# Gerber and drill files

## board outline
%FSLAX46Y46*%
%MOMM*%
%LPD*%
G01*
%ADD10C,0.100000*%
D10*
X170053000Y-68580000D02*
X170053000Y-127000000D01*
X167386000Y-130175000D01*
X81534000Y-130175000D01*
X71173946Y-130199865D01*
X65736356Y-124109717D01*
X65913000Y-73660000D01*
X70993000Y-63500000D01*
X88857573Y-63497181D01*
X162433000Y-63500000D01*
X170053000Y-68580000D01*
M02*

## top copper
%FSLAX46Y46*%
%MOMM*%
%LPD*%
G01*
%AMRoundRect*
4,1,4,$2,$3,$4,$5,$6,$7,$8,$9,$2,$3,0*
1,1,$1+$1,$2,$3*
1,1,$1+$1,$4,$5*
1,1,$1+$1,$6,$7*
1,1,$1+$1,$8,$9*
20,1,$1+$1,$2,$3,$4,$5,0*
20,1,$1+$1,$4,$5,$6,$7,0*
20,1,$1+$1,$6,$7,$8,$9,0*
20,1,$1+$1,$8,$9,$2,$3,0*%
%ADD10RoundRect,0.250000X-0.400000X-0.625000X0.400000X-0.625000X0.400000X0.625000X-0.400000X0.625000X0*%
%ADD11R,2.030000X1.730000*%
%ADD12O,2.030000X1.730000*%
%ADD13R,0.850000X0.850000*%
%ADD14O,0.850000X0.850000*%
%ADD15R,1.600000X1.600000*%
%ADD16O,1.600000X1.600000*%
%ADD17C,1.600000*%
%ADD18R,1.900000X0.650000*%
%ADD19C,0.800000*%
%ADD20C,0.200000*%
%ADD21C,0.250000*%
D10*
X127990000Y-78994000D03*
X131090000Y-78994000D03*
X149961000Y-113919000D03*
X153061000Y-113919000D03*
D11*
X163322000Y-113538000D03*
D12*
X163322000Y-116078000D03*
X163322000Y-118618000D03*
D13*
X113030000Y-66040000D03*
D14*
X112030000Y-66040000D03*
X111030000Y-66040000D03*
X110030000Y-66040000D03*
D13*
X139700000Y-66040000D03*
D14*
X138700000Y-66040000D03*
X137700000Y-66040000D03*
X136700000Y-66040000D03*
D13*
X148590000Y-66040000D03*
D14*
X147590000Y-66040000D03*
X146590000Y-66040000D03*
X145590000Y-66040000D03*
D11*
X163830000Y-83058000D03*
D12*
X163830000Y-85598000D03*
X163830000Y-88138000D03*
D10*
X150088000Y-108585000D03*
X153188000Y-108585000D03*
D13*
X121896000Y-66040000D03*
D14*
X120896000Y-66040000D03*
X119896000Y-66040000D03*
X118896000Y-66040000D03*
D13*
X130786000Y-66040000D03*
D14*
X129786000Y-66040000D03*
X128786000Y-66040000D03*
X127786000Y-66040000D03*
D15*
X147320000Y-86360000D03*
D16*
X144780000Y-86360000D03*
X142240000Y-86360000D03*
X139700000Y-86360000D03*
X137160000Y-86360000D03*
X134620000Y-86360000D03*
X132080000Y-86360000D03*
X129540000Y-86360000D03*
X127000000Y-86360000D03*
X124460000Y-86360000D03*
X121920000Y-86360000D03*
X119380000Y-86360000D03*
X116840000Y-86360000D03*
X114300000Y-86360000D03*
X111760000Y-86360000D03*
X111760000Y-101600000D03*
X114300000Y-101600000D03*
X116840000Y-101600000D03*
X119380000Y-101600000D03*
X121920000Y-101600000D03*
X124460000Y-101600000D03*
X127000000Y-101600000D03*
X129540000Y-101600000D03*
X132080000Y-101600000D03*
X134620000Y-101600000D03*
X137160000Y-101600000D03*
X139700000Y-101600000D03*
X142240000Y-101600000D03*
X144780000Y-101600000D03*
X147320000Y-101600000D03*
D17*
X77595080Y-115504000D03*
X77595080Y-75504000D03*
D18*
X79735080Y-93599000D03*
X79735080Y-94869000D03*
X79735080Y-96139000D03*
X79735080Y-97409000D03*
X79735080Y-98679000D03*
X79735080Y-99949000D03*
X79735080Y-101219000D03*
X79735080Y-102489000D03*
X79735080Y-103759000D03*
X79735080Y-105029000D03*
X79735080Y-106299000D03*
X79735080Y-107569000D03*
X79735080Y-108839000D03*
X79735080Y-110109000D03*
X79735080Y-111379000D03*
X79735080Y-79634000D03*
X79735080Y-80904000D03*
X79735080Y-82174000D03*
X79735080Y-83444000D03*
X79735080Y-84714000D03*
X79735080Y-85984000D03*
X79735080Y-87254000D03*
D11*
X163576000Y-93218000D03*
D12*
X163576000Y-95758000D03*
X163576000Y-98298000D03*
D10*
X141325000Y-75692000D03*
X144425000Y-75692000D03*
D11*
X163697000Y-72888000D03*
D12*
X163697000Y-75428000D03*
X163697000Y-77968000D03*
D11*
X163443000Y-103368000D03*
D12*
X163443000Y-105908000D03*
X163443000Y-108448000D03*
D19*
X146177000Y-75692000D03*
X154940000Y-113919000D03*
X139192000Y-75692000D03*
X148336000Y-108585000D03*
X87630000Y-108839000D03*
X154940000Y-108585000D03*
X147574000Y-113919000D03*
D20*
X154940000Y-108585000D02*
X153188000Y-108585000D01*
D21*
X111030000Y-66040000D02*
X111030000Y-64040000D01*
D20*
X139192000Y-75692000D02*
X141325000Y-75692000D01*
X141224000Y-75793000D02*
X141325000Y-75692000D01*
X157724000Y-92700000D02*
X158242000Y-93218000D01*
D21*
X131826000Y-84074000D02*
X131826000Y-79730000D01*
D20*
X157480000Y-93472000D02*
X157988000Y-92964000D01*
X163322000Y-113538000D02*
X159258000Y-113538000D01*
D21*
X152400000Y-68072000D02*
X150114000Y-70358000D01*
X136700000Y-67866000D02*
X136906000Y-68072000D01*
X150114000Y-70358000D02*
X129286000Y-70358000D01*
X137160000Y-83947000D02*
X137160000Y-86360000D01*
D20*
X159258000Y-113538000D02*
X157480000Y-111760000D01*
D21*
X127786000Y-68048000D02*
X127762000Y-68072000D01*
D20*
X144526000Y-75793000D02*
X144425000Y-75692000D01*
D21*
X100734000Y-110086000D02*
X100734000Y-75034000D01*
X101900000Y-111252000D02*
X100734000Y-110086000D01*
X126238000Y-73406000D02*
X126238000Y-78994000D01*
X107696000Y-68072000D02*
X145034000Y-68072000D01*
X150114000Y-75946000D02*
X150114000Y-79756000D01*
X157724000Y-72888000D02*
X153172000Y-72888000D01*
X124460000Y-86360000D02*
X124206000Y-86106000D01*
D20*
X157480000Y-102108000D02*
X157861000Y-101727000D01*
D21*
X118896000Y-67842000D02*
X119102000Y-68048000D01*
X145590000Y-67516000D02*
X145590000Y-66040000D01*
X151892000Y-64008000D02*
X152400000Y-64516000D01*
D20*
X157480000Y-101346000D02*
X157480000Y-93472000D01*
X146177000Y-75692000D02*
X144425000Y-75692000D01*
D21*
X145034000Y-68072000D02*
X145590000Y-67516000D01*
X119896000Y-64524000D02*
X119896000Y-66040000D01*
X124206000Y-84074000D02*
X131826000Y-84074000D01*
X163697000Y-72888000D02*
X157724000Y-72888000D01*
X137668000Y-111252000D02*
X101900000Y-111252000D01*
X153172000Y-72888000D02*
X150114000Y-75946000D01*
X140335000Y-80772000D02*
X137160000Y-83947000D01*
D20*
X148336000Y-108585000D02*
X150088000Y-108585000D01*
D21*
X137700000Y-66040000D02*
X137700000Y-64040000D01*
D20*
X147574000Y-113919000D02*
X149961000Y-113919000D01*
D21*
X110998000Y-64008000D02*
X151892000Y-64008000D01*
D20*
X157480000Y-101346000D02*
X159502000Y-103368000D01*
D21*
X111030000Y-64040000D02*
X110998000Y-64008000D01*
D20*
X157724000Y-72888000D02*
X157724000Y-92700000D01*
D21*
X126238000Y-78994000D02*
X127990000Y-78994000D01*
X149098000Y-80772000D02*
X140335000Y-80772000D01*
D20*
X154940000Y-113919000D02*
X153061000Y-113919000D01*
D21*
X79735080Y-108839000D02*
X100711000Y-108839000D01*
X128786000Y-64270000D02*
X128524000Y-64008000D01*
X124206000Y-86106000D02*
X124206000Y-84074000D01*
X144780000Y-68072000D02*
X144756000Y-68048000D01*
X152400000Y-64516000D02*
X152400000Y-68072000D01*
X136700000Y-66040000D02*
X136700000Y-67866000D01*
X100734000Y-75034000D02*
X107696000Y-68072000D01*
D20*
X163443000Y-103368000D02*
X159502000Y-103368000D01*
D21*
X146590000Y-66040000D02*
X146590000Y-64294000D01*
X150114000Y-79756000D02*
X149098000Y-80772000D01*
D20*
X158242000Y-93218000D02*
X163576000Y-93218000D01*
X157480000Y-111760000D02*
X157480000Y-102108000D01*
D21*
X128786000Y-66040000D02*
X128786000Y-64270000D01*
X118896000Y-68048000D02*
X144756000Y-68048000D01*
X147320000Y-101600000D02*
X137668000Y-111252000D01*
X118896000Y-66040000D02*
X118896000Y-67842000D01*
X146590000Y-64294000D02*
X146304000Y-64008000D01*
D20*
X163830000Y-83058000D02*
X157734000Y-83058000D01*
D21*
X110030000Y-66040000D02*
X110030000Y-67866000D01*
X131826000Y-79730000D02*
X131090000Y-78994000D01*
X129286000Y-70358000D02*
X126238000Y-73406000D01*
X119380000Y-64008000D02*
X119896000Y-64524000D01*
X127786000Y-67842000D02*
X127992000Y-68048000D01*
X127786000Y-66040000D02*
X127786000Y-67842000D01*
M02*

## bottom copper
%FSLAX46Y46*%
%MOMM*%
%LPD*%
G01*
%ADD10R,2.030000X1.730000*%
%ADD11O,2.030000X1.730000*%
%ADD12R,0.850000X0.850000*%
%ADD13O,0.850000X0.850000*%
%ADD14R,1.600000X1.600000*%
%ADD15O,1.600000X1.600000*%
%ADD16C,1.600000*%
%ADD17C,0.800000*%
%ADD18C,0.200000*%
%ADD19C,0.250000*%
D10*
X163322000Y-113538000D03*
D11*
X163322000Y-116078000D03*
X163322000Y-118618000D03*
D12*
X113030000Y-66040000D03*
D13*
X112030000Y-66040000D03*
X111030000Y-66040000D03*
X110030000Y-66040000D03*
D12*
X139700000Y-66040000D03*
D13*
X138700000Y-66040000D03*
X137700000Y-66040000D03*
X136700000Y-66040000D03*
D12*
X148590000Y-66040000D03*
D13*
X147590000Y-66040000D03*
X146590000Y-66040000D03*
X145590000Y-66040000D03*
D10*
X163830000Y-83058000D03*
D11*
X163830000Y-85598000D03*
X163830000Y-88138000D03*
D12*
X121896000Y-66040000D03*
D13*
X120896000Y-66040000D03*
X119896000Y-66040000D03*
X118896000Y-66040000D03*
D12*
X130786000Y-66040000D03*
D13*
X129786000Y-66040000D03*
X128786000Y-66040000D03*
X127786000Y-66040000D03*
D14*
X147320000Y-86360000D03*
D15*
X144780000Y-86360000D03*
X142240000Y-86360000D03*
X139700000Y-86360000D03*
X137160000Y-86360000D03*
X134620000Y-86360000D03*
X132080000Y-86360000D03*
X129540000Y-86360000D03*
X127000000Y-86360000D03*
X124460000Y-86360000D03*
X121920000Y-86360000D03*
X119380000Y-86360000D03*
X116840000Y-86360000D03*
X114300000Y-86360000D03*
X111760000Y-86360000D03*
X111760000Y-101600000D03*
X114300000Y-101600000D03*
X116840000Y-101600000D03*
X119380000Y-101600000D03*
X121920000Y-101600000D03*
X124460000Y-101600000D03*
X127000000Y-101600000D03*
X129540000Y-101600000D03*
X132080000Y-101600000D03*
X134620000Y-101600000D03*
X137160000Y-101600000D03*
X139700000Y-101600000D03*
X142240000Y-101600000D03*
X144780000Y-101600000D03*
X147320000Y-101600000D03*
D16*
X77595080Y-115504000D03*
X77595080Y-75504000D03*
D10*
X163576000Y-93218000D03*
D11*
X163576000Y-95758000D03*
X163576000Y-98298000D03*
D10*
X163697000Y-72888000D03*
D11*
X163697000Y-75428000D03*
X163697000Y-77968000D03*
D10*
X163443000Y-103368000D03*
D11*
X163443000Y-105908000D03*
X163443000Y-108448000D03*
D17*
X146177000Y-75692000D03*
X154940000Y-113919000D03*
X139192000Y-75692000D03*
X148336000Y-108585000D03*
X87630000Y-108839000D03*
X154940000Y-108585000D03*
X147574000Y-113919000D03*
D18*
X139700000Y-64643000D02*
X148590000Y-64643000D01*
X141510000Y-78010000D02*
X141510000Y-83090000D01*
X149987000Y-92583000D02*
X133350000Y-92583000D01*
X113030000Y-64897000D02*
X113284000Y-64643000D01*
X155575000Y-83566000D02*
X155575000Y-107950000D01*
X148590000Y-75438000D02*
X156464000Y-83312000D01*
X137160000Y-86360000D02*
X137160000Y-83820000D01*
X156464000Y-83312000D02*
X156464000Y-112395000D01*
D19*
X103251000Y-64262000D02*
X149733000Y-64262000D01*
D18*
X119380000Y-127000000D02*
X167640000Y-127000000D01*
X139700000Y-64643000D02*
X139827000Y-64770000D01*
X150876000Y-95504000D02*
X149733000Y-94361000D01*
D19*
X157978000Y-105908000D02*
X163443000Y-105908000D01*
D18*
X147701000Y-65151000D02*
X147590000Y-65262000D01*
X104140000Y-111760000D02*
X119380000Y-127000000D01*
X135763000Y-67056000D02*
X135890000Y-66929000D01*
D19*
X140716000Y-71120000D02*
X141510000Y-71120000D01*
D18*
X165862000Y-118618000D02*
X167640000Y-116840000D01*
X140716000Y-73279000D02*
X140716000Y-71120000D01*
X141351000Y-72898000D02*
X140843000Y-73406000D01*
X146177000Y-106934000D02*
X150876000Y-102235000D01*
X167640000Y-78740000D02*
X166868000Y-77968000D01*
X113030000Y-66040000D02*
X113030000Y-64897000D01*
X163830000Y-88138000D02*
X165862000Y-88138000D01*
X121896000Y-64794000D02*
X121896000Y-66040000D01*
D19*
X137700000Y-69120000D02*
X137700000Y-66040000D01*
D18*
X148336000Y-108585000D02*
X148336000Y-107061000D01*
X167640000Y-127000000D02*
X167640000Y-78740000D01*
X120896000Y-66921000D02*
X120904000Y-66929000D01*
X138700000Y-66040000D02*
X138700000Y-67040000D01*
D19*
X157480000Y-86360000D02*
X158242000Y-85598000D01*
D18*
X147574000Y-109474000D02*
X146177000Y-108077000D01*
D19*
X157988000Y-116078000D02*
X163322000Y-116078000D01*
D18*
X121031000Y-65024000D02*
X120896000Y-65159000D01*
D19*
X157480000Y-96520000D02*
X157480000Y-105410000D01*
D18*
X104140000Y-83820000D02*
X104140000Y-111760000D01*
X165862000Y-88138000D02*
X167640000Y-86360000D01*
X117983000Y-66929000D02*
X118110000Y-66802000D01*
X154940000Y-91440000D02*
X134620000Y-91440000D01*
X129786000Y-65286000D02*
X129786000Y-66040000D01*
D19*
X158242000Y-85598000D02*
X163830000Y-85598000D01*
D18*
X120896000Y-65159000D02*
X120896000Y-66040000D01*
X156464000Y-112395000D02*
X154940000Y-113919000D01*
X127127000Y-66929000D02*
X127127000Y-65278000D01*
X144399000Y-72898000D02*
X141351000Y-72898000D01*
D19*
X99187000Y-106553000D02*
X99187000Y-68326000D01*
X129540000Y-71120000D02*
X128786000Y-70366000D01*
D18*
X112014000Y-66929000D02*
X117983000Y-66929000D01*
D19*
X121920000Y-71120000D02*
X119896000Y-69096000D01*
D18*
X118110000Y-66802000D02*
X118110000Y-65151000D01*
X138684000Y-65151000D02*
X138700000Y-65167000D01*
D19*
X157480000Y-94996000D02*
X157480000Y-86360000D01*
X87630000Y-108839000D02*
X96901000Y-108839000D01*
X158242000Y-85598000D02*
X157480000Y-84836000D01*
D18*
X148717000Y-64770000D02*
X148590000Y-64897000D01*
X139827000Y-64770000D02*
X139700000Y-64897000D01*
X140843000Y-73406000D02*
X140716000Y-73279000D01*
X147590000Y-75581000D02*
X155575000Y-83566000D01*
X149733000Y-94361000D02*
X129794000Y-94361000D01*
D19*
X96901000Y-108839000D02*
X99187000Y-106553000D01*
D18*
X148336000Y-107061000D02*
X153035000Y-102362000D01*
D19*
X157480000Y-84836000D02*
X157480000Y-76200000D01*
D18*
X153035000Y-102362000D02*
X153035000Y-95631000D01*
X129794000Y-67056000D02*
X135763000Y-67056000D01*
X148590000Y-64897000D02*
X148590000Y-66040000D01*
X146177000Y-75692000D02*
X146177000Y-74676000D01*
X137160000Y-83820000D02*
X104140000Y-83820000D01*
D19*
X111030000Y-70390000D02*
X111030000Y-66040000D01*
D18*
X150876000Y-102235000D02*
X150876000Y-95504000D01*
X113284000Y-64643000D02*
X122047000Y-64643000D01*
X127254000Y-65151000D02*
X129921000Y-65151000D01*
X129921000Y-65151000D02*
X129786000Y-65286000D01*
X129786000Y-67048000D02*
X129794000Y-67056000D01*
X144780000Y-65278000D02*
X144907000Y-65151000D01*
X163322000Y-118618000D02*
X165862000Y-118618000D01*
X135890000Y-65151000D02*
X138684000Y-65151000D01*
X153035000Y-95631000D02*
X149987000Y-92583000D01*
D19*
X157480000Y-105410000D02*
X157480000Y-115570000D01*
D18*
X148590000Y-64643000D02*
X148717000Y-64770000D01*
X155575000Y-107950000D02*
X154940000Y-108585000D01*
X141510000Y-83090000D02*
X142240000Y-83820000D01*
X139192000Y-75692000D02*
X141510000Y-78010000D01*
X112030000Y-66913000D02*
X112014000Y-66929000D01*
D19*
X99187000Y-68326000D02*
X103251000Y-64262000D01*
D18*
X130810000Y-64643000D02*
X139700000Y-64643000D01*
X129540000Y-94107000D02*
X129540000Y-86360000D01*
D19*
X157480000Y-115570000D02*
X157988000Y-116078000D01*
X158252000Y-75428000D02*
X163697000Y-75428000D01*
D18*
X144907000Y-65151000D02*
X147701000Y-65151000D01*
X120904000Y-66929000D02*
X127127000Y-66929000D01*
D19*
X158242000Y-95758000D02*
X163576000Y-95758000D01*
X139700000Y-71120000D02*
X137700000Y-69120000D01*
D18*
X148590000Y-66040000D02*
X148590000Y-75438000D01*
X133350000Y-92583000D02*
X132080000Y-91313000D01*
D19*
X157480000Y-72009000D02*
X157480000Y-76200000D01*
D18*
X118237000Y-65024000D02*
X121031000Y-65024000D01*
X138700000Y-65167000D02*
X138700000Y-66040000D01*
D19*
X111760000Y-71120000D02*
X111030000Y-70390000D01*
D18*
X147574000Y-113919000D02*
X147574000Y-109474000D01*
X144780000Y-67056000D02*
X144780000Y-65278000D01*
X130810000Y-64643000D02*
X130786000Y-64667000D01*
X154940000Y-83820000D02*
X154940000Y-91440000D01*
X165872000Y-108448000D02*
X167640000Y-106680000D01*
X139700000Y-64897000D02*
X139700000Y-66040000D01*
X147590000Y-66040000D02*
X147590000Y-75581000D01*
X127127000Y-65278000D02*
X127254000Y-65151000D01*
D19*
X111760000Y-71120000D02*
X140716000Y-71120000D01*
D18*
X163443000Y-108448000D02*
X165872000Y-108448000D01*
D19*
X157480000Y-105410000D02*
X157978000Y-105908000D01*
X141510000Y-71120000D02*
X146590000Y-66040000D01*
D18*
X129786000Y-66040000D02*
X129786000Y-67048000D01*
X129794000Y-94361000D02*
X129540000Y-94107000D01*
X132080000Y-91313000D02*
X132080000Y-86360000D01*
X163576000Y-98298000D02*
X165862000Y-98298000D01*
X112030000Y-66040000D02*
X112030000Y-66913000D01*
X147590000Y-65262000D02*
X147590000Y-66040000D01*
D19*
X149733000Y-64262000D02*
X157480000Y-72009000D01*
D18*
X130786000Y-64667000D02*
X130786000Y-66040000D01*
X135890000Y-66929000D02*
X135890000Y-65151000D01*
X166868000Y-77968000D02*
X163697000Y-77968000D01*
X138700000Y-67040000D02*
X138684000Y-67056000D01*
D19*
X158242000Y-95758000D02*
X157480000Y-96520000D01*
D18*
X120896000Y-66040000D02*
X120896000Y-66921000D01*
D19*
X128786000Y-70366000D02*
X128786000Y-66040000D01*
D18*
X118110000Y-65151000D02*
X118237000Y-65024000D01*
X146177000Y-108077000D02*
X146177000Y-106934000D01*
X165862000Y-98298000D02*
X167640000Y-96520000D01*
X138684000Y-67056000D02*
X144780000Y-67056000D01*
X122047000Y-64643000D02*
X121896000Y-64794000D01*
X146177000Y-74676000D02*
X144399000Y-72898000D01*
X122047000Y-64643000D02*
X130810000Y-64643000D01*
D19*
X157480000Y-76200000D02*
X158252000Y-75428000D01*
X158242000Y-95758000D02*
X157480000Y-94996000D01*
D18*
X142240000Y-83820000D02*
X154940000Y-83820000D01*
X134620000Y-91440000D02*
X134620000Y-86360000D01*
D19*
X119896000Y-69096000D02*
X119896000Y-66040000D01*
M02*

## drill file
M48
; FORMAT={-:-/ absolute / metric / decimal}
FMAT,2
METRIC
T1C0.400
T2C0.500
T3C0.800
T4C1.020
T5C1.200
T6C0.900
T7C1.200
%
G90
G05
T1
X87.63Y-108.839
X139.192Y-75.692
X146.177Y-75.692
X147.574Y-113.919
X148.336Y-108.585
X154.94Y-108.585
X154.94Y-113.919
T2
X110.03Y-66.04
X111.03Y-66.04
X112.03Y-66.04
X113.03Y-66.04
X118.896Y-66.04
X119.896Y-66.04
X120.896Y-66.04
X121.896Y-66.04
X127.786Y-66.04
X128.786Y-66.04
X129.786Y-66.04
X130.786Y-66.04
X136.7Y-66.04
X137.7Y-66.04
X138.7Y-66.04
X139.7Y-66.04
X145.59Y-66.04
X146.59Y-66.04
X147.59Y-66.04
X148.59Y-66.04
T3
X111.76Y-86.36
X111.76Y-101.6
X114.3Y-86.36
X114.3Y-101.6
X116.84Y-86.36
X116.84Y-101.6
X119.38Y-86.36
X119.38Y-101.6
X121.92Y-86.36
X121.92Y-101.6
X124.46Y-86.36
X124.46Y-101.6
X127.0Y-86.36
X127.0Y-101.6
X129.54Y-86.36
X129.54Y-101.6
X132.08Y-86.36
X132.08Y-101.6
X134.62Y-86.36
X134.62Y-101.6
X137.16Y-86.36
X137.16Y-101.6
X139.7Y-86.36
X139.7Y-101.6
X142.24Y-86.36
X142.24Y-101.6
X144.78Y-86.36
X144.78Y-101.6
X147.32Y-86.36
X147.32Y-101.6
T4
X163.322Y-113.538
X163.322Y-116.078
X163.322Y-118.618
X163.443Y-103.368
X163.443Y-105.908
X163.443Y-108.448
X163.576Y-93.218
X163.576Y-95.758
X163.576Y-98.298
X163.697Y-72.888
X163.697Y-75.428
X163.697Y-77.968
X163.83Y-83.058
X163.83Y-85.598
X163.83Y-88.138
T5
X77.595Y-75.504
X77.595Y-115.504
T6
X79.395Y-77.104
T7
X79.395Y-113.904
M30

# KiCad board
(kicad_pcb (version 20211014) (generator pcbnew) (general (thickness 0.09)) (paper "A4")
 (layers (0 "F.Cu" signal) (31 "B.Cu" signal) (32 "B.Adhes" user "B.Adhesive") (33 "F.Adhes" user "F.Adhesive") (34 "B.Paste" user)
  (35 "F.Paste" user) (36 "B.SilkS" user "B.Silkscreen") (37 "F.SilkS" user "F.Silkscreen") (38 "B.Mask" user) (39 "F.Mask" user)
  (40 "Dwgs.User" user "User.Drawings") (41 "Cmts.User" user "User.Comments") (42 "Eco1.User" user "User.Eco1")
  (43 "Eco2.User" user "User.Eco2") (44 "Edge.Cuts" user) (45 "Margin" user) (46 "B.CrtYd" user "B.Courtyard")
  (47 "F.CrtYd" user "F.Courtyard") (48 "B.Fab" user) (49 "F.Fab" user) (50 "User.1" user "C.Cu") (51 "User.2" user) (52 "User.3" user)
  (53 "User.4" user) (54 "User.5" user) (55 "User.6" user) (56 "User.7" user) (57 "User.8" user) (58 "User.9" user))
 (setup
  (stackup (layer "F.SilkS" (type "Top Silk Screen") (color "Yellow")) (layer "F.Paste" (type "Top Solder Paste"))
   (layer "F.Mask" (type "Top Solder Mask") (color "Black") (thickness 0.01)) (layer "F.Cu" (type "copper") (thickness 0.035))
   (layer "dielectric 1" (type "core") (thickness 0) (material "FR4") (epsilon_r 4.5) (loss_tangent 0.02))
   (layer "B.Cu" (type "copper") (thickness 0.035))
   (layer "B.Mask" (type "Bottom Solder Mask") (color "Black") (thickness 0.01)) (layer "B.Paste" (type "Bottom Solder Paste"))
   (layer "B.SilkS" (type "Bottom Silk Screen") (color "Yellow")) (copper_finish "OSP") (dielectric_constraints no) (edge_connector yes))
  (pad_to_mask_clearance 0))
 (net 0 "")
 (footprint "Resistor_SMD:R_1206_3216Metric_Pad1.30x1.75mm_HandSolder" (layer "F.Cu") (at 129.54 78.994)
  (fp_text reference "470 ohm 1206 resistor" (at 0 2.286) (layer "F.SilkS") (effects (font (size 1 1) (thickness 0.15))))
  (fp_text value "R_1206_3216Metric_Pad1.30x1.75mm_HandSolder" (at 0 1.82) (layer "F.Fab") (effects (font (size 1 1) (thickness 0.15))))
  (pad "1" smd roundrect (at -1.55 0) (size 1.3 1.75) (layers "F.Cu" "F.Paste" "F.Mask") (roundrect_rratio 0.1923076923))
  (pad "2" smd roundrect (at 1.55 0) (size 1.3 1.75) (layers "F.Cu" "F.Paste" "F.Mask") (roundrect_rratio 0.1923076923)))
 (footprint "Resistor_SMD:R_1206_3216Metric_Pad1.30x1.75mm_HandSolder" (layer "F.Cu") (at 151.511 113.919)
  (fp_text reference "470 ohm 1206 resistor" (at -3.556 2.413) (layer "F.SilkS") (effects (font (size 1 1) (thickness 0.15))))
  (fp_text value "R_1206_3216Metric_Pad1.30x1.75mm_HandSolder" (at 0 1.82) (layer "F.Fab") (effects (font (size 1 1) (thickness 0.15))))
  (pad "1" smd roundrect (at -1.55 0) (size 1.3 1.75) (layers "F.Cu" "F.Paste" "F.Mask") (roundrect_rratio 0.1923076923))
  (pad "2" smd roundrect (at 1.55 0) (size 1.3 1.75) (layers "F.Cu" "F.Paste" "F.Mask") (roundrect_rratio 0.1923076923)))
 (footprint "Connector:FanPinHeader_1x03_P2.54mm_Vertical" (layer "F.Cu") (at 163.322 113.538 -90)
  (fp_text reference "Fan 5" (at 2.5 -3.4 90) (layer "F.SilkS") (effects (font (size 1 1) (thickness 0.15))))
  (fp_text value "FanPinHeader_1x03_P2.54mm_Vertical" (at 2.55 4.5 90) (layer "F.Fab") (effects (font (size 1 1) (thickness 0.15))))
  (pad "1" thru_hole rect (at 0 0) (size 2.03 1.73) (drill 1.02) (layers *.Cu *.Mask))
  (pad "2" thru_hole oval (at 2.54 0) (size 2.03 1.73) (drill 1.02) (layers *.Cu *.Mask))
  (pad "3" thru_hole oval (at 5.08 0) (size 2.03 1.73) (drill 1.02) (layers *.Cu *.Mask)))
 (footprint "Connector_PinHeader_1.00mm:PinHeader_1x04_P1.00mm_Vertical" (layer "F.Cu") (at 113.03 66.04 -90)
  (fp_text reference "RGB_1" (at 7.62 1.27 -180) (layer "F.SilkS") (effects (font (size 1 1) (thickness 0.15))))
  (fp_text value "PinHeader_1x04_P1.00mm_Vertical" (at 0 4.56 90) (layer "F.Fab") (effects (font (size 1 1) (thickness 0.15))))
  (pad "1" thru_hole rect (at 0 0 270) (size 0.85 0.85) (drill 0.5) (layers *.Cu *.Mask))
  (pad "2" thru_hole oval (at 0 1 270) (size 0.85 0.85) (drill 0.5) (layers *.Cu *.Mask))
  (pad "3" thru_hole oval (at 0 2 270) (size 0.85 0.85) (drill 0.5) (layers *.Cu *.Mask))
  (pad "4" thru_hole oval (at 0 3 270) (size 0.85 0.85) (drill 0.5) (layers *.Cu *.Mask)))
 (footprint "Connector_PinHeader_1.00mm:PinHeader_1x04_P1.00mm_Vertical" (layer "F.Cu") (at 139.7 66.04 -90)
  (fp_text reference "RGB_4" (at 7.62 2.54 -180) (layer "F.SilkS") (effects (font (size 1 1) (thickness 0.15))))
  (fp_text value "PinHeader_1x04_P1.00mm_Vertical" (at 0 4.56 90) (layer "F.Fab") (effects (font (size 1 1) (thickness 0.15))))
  (pad "1" thru_hole rect (at 0 0 270) (size 0.85 0.85) (drill 0.5) (layers *.Cu *.Mask))
  (pad "2" thru_hole oval (at 0 1 270) (size 0.85 0.85) (drill 0.5) (layers *.Cu *.Mask))
  (pad "3" thru_hole oval (at 0 2 270) (size 0.85 0.85) (drill 0.5) (layers *.Cu *.Mask))
  (pad "4" thru_hole oval (at 0 3 270) (size 0.85 0.85) (drill 0.5) (layers *.Cu *.Mask)))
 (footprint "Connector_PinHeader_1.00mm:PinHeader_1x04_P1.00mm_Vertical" (layer "F.Cu") (at 148.59 66.04 -90)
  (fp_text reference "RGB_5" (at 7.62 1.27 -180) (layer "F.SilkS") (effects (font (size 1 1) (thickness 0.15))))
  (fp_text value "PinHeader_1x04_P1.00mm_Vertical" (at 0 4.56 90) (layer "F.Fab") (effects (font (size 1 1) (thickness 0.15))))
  (pad "1" thru_hole rect (at 0 0 270) (size 0.85 0.85) (drill 0.5) (layers *.Cu *.Mask))
  (pad "2" thru_hole oval (at 0 1 270) (size 0.85 0.85) (drill 0.5) (layers *.Cu *.Mask))
  (pad "3" thru_hole oval (at 0 2 270) (size 0.85 0.85) (drill 0.5) (layers *.Cu *.Mask))
  (pad "4" thru_hole oval (at 0 3 270) (size 0.85 0.85) (drill 0.5) (layers *.Cu *.Mask)))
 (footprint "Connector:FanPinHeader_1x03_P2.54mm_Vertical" (layer "F.Cu") (at 163.83 83.058 -90)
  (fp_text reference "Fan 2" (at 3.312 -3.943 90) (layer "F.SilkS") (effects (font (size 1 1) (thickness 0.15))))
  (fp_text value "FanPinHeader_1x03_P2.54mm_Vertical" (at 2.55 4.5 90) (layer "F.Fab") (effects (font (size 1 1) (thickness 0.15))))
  (pad "1" thru_hole rect (at 0 0) (size 2.03 1.73) (drill 1.02) (layers *.Cu *.Mask))
  (pad "2" thru_hole oval (at 2.54 0) (size 2.03 1.73) (drill 1.02) (layers *.Cu *.Mask))
  (pad "3" thru_hole oval (at 5.08 0) (size 2.03 1.73) (drill 1.02) (layers *.Cu *.Mask)))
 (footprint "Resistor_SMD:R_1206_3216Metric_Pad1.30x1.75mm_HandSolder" (layer "F.Cu") (at 151.638 108.585)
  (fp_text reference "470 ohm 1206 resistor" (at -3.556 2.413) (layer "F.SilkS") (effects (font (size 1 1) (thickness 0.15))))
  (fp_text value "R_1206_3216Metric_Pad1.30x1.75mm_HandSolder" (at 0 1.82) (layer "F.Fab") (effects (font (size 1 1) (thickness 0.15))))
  (pad "1" smd roundrect (at -1.55 0) (size 1.3 1.75) (layers "F.Cu" "F.Paste" "F.Mask") (roundrect_rratio 0.1923076923))
  (pad "2" smd roundrect (at 1.55 0) (size 1.3 1.75) (layers "F.Cu" "F.Paste" "F.Mask") (roundrect_rratio 0.1923076923)))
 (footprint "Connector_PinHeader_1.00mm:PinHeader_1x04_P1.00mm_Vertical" (layer "F.Cu") (at 121.896 66.04 -90)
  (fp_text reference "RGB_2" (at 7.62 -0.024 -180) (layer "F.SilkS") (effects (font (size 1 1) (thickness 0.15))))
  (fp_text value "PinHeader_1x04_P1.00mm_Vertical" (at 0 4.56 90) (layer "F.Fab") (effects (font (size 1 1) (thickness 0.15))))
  (pad "1" thru_hole rect (at 0 0 270) (size 0.85 0.85) (drill 0.5) (layers *.Cu *.Mask))
  (pad "2" thru_hole oval (at 0 1 270) (size 0.85 0.85) (drill 0.5) (layers *.Cu *.Mask))
  (pad "3" thru_hole oval (at 0 2 270) (size 0.85 0.85) (drill 0.5) (layers *.Cu *.Mask))
  (pad "4" thru_hole oval (at 0 3 270) (size 0.85 0.85) (drill 0.5) (layers *.Cu *.Mask)))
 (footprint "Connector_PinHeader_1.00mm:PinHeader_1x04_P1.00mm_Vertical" (layer "F.Cu") (at 130.786 66.04 -90)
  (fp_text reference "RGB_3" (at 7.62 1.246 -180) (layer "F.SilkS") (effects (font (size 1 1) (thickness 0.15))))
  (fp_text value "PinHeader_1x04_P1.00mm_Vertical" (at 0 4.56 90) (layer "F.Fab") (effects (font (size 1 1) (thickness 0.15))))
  (pad "1" thru_hole rect (at 0 0 270) (size 0.85 0.85) (drill 0.5) (layers *.Cu *.Mask))
  (pad "2" thru_hole oval (at 0 1 270) (size 0.85 0.85) (drill 0.5) (layers *.Cu *.Mask))
  (pad "3" thru_hole oval (at 0 2 270) (size 0.85 0.85) (drill 0.5) (layers *.Cu *.Mask))
  (pad "4" thru_hole oval (at 0 3 270) (size 0.85 0.85) (drill 0.5) (layers *.Cu *.Mask)))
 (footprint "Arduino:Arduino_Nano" (layer "F.Cu") (at 147.32 86.36 -90)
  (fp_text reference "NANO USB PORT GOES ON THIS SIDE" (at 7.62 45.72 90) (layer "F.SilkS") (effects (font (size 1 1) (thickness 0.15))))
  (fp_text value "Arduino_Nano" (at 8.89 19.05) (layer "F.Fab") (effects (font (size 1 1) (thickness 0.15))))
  (pad "1" thru_hole rect locked (at 0 0 270) (size 1.6 1.6) (drill 0.8) (layers *.Cu *.Mask))
  (pad "2" thru_hole oval locked (at 0 2.54 270) (size 1.6 1.6) (drill 0.8) (layers *.Cu *.Mask))
  (pad "3" thru_hole oval locked (at 0 5.08 270) (size 1.6 1.6) (drill 0.8) (layers *.Cu *.Mask))
  (pad "4" thru_hole oval locked (at 0 7.62 270) (size 1.6 1.6) (drill 0.8) (layers *.Cu *.Mask))
  (pad "5" thru_hole oval locked (at 0 10.16 270) (size 1.6 1.6) (drill 0.8) (layers *.Cu *.Mask))
  (pad "6" thru_hole oval locked (at 0 12.7 270) (size 1.6 1.6) (drill 0.8) (layers *.Cu *.Mask))
  (pad "7" thru_hole oval locked (at 0 15.24 270) (size 1.6 1.6) (drill 0.8) (layers *.Cu *.Mask))
  (pad "8" thru_hole oval locked (at 0 17.78 270) (size 1.6 1.6) (drill 0.8) (layers *.Cu *.Mask))
  (pad "9" thru_hole oval locked (at 0 20.32 270) (size 1.6 1.6) (drill 0.8) (layers *.Cu *.Mask))
  (pad "10" thru_hole oval locked (at 0 22.86 270) (size 1.6 1.6) (drill 0.8) (layers *.Cu *.Mask))
  (pad "11" thru_hole oval locked (at 0 25.4 270) (size 1.6 1.6) (drill 0.8) (layers *.Cu *.Mask))
  (pad "12" thru_hole oval locked (at 0 27.94 270) (size 1.6 1.6) (drill 0.8) (layers *.Cu *.Mask))
  (pad "13" thru_hole oval locked (at 0 30.48 270) (size 1.6 1.6) (drill 0.8) (layers *.Cu *.Mask))
  (pad "14" thru_hole oval locked (at 0 33.02 270) (size 1.6 1.6) (drill 0.8) (layers *.Cu *.Mask))
  (pad "15" thru_hole oval locked (at 0 35.56 270) (size 1.6 1.6) (drill 0.8) (layers *.Cu *.Mask))
  (pad "16" thru_hole oval locked (at 15.24 35.56 270) (size 1.6 1.6) (drill 0.8) (layers *.Cu *.Mask))
  (pad "17" thru_hole oval locked (at 15.24 33.02 270) (size 1.6 1.6) (drill 0.8) (layers *.Cu *.Mask))
  (pad "18" thru_hole oval locked (at 15.24 30.48 270) (size 1.6 1.6) (drill 0.8) (layers *.Cu *.Mask))
  (pad "19" thru_hole oval locked (at 15.24 27.94 270) (size 1.6 1.6) (drill 0.8) (layers *.Cu *.Mask))
  (pad "20" thru_hole oval locked (at 15.24 25.4 270) (size 1.6 1.6) (drill 0.8) (layers *.Cu *.Mask))
  (pad "21" thru_hole oval locked (at 15.24 22.86 270) (size 1.6 1.6) (drill 0.8) (layers *.Cu *.Mask))
  (pad "22" thru_hole oval locked (at 15.24 20.32 270) (size 1.6 1.6) (drill 0.8) (layers *.Cu *.Mask))
  (pad "23" thru_hole oval locked (at 15.24 17.78 270) (size 1.6 1.6) (drill 0.8) (layers *.Cu *.Mask))
  (pad "24" thru_hole oval locked (at 15.24 15.24 270) (size 1.6 1.6) (drill 0.8) (layers *.Cu *.Mask))
  (pad "25" thru_hole oval locked (at 15.24 12.7 270) (size 1.6 1.6) (drill 0.8) (layers *.Cu *.Mask))
  (pad "26" thru_hole oval locked (at 15.24 10.16 270) (size 1.6 1.6) (drill 0.8) (layers *.Cu *.Mask))
  (pad "27" thru_hole oval locked (at 15.24 7.62 270) (size 1.6 1.6) (drill 0.8) (layers *.Cu *.Mask))
  (pad "28" thru_hole oval locked (at 15.24 5.08 270) (size 1.6 1.6) (drill 0.8) (layers *.Cu *.Mask))
  (pad "29" thru_hole oval locked (at 15.24 2.54 270) (size 1.6 1.6) (drill 0.8) (layers *.Cu *.Mask))
  (pad "30" thru_hole oval locked (at 15.24 0 270) (size 1.6 1.6) (drill 0.8) (layers *.Cu *.Mask)))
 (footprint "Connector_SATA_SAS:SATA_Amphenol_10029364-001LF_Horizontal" (layer "F.Cu") (at 78.74 95.504 90)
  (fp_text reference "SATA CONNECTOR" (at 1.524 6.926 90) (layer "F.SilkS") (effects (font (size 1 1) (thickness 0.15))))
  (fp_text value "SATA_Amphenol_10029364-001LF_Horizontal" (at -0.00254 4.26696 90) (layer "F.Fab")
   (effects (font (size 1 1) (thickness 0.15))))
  (pad "" np_thru_hole circle (at -18.4 0.65508 90) (size 1.2 1.2) (drill 1.2) (layers *.Mask "B.Cu"))
  (pad "" np_thru_hole circle (at 18.4 0.65508 90) (size 0.9 0.9) (drill 0.9) (layers *.Mask "B.Cu"))
  (pad "MP" thru_hole circle (at -20 -1.14492 90) (size 1.6 1.6) (drill 1.2) (layers *.Cu *.Mask) (zone_connect 2))
  (pad "MP" thru_hole circle (at 20 -1.14492 90) (size 1.6 1.6) (drill 1.2) (layers *.Cu *.Mask))
  (pad "P1" smd rect (at 1.905 0.99508 90) (size 0.65 1.9) (layers "F.Cu" "F.Paste" "F.Mask"))
  (pad "P2" smd rect (at 0.635 0.99508 90) (size 0.65 1.9) (layers "F.Cu" "F.Paste" "F.Mask"))
  (pad "P3" smd rect (at -0.635 0.99508 90) (size 0.65 1.9) (layers "F.Cu" "F.Paste" "F.Mask"))
  (pad "P4" smd rect (at -1.905 0.99508 90) (size 0.65 1.9) (layers "F.Cu" "F.Paste" "F.Mask"))
  (pad "P5" smd rect (at -3.175 0.99508 90) (size 0.65 1.9) (layers "F.Cu" "F.Paste" "F.Mask"))
  (pad "P6" smd rect (at -4.445 0.99508 90) (size 0.65 1.9) (layers "F.Cu" "F.Paste" "F.Mask"))
  (pad "P7" smd rect (at -5.715 0.99508 90) (size 0.65 1.9) (layers "F.Cu" "F.Paste" "F.Mask"))
  (pad "P8" smd rect (at -6.985 0.99508 90) (size 0.65 1.9) (layers "F.Cu" "F.Paste" "F.Mask"))
  (pad "P9" smd rect (at -8.255 0.99508 90) (size 0.65 1.9) (layers "F.Cu" "F.Paste" "F.Mask"))
  (pad "P10" smd rect (at -9.525 0.99508 90) (size 0.65 1.9) (layers "F.Cu" "F.Paste" "F.Mask"))
  (pad "P11" smd rect (at -10.795 0.99508 90) (size 0.65 1.9) (layers "F.Cu" "F.Paste" "F.Mask"))
  (pad "P12" smd rect (at -12.065 0.99508 90) (size 0.65 1.9) (layers "F.Cu" "F.Paste" "F.Mask"))
  (pad "P13" smd rect (at -13.335 0.99508 90) (size 0.65 1.9) (layers "F.Cu" "F.Paste" "F.Mask"))
  (pad "P14" smd rect (at -14.605 0.99508 90) (size 0.65 1.9) (layers "F.Cu" "F.Paste" "F.Mask"))
  (pad "P15" smd rect (at -15.875 0.99508 90) (size 0.65 1.9) (layers "F.Cu" "F.Paste" "F.Mask"))
  (pad "S1" smd rect (at 15.87 0.99508 90) (size 0.65 1.9) (layers "F.Cu" "F.Paste" "F.Mask"))
  (pad "S2" smd rect (at 14.6 0.99508 90) (size 0.65 1.9) (layers "F.Cu" "F.Paste" "F.Mask"))
  (pad "S3" smd rect (at 13.33 0.99508 90) (size 0.65 1.9) (layers "F.Cu" "F.Paste" "F.Mask"))
  (pad "S4" smd rect (at 12.06 0.99508 90) (size 0.65 1.9) (layers "F.Cu" "F.Paste" "F.Mask"))
  (pad "S5" smd rect (at 10.79 0.99508 90) (size 0.65 1.9) (layers "F.Cu" "F.Paste" "F.Mask"))
  (pad "S6" smd rect (at 9.52 0.99508 90) (size 0.65 1.9) (layers "F.Cu" "F.Paste" "F.Mask"))
  (pad "S7" smd rect (at 8.25 0.99508 90) (size 0.65 1.9) (layers "F.Cu" "F.Paste" "F.Mask")))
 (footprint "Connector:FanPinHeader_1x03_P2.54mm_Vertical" (layer "F.Cu") (at 163.576 93.218 -90)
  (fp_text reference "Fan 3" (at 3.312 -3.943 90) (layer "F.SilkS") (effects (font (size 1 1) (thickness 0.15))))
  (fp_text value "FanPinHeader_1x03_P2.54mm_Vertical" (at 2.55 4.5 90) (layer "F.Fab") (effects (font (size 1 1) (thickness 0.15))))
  (pad "1" thru_hole rect (at 0 0) (size 2.03 1.73) (drill 1.02) (layers *.Cu *.Mask))
  (pad "2" thru_hole oval (at 2.54 0) (size 2.03 1.73) (drill 1.02) (layers *.Cu *.Mask))
  (pad "3" thru_hole oval (at 5.08 0) (size 2.03 1.73) (drill 1.02) (layers *.Cu *.Mask)))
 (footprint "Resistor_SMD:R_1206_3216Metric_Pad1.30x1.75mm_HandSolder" (layer "F.Cu") (at 142.875 75.692)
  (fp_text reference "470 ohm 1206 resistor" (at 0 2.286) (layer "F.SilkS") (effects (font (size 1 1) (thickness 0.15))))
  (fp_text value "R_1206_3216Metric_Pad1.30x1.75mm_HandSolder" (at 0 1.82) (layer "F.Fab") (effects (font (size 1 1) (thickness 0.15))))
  (pad "1" smd roundrect (at -1.55 0) (size 1.3 1.75) (layers "F.Cu" "F.Paste" "F.Mask") (roundrect_rratio 0.1923076923))
  (pad "2" smd roundrect (at 1.55 0) (size 1.3 1.75) (layers "F.Cu" "F.Paste" "F.Mask") (roundrect_rratio 0.1923076923)))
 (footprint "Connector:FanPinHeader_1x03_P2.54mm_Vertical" (layer "F.Cu") (at 163.697 72.888 -90)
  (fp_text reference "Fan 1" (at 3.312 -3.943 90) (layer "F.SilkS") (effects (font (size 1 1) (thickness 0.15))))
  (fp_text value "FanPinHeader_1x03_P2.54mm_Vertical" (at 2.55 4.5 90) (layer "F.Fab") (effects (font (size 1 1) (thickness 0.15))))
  (pad "1" thru_hole rect (at 0 0) (size 2.03 1.73) (drill 1.02) (layers *.Cu *.Mask))
  (pad "2" thru_hole oval (at 2.54 0) (size 2.03 1.73) (drill 1.02) (layers *.Cu *.Mask))
  (pad "3" thru_hole oval (at 5.08 0) (size 2.03 1.73) (drill 1.02) (layers *.Cu *.Mask)))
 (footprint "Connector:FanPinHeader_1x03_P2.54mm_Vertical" (layer "F.Cu") (at 163.443 103.368 -90)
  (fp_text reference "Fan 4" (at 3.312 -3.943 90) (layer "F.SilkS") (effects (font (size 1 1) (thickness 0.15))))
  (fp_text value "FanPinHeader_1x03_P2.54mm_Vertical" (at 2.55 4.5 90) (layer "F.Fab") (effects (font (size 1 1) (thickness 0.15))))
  (pad "1" thru_hole rect (at 0 0) (size 2.03 1.73) (drill 1.02) (layers *.Cu *.Mask))
  (pad "2" thru_hole oval (at 2.54 0) (size 2.03 1.73) (drill 1.02) (layers *.Cu *.Mask))
  (pad "3" thru_hole oval (at 5.08 0) (size 2.03 1.73) (drill 1.02) (layers *.Cu *.Mask)))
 (gr_poly
  (pts (xy 170.053 68.58) (xy 170.053 127) (xy 167.386 130.175) (xy 81.534 130.175) (xy 71.173946 130.199865) (xy 65.736356 124.109717)
   (xy 65.913 73.66) (xy 70.993 63.5) (xy 88.857573 63.497181) (xy 162.433 63.5))
  (layer "Edge.Cuts") (width 0.1) (fill none))
 (segment (start 154.94 108.585) (end 153.188 108.585) (width 0.2) (layer "F.Cu") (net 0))
 (segment (start 111.03 66.04) (end 111.03 64.04) (width 0.25) (layer "F.Cu") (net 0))
 (segment (start 139.192 75.692) (end 141.325 75.692) (width 0.2) (layer "F.Cu") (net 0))
 (segment (start 141.224 75.793) (end 141.325 75.692) (width 0.2) (layer "F.Cu") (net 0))
 (segment (start 157.724 92.7) (end 158.242 93.218) (width 0.2) (layer "F.Cu") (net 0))
 (segment (start 131.826 84.074) (end 131.826 79.73) (width 0.25) (layer "F.Cu") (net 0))
 (segment (start 157.48 93.472) (end 157.988 92.964) (width 0.2) (layer "F.Cu") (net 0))
 (segment (start 163.322 113.538) (end 159.258 113.538) (width 0.2) (layer "F.Cu") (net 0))
 (segment (start 152.4 68.072) (end 150.114 70.358) (width 0.25) (layer "F.Cu") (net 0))
 (segment (start 136.7 67.866) (end 136.906 68.072) (width 0.25) (layer "F.Cu") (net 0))
 (segment (start 150.114 70.358) (end 129.286 70.358) (width 0.25) (layer "F.Cu") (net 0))
 (segment (start 137.16 83.947) (end 137.16 86.36) (width 0.25) (layer "F.Cu") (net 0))
 (segment (start 159.258 113.538) (end 157.48 111.76) (width 0.2) (layer "F.Cu") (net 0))
 (segment (start 127.786 68.048) (end 127.762 68.072) (width 0.25) (layer "F.Cu") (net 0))
 (segment (start 144.526 75.793) (end 144.425 75.692) (width 0.2) (layer "F.Cu") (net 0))
 (segment (start 100.734 110.086) (end 100.734 75.034) (width 0.25) (layer "F.Cu") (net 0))
 (segment (start 101.9 111.252) (end 100.734 110.086) (width 0.25) (layer "F.Cu") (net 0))
 (segment (start 126.238 73.406) (end 126.238 78.994) (width 0.25) (layer "F.Cu") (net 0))
 (segment (start 107.696 68.072) (end 145.034 68.072) (width 0.25) (layer "F.Cu") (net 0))
 (segment (start 150.114 75.946) (end 150.114 79.756) (width 0.25) (layer "F.Cu") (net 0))
 (segment (start 157.724 72.888) (end 153.172 72.888) (width 0.25) (layer "F.Cu") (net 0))
 (segment (start 124.46 86.36) (end 124.206 86.106) (width 0.25) (layer "F.Cu") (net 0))
 (segment (start 157.48 102.108) (end 157.861 101.727) (width 0.2) (layer "F.Cu") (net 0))
 (segment (start 118.896 67.842) (end 119.102 68.048) (width 0.25) (layer "F.Cu") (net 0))
 (segment (start 145.59 67.516) (end 145.59 66.04) (width 0.25) (layer "F.Cu") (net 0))
 (segment (start 151.892 64.008) (end 152.4 64.516) (width 0.25) (layer "F.Cu") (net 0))
 (segment (start 157.48 101.346) (end 157.48 93.472) (width 0.2) (layer "F.Cu") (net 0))
 (segment (start 146.177 75.692) (end 144.425 75.692) (width 0.2) (layer "F.Cu") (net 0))
 (segment (start 145.034 68.072) (end 145.59 67.516) (width 0.25) (layer "F.Cu") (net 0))
 (segment (start 119.896 64.524) (end 119.896 66.04) (width 0.25) (layer "F.Cu") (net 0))
 (segment (start 124.206 84.074) (end 131.826 84.074) (width 0.25) (layer "F.Cu") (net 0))
 (segment (start 163.697 72.888) (end 157.724 72.888) (width 0.25) (layer "F.Cu") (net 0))
 (segment (start 137.668 111.252) (end 101.9 111.252) (width 0.25) (layer "F.Cu") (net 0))
 (segment (start 153.172 72.888) (end 150.114 75.946) (width 0.25) (layer "F.Cu") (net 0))
 (segment (start 140.335 80.772) (end 137.16 83.947) (width 0.25) (layer "F.Cu") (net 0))
 (segment (start 148.336 108.585) (end 150.088 108.585) (width 0.2) (layer "F.Cu") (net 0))
 (segment (start 137.7 66.04) (end 137.7 64.04) (width 0.25) (layer "F.Cu") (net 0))
 (segment (start 147.574 113.919) (end 149.961 113.919) (width 0.2) (layer "F.Cu") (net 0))
 (segment (start 110.998 64.008) (end 151.892 64.008) (width 0.25) (layer "F.Cu") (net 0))
 (segment (start 157.48 101.346) (end 159.502 103.368) (width 0.2) (layer "F.Cu") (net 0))
 (segment (start 111.03 64.04) (end 110.998 64.008) (width 0.25) (layer "F.Cu") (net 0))
 (segment (start 157.724 72.888) (end 157.724 92.7) (width 0.2) (layer "F.Cu") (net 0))
 (segment (start 126.238 78.994) (end 127.99 78.994) (width 0.25) (layer "F.Cu") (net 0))
 (segment (start 149.098 80.772) (end 140.335 80.772) (width 0.25) (layer "F.Cu") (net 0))
 (segment (start 154.94 113.919) (end 153.061 113.919) (width 0.2) (layer "F.Cu") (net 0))
 (segment (start 79.73508 108.839) (end 100.711 108.839) (width 0.25) (layer "F.Cu") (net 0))
 (segment (start 128.786 64.27) (end 128.524 64.008) (width 0.25) (layer "F.Cu") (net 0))
 (segment (start 124.206 86.106) (end 124.206 84.074) (width 0.25) (layer "F.Cu") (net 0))
 (segment (start 144.78 68.072) (end 144.756 68.048) (width 0.25) (layer "F.Cu") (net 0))
 (segment (start 152.4 64.516) (end 152.4 68.072) (width 0.25) (layer "F.Cu") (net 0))
 (segment (start 136.7 66.04) (end 136.7 67.866) (width 0.25) (layer "F.Cu") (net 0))
 (segment (start 100.734 75.034) (end 107.696 68.072) (width 0.25) (layer "F.Cu") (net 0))
 (segment (start 163.443 103.368) (end 159.502 103.368) (width 0.2) (layer "F.Cu") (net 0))
 (segment (start 146.59 66.04) (end 146.59 64.294) (width 0.25) (layer "F.Cu") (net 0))
 (segment (start 150.114 79.756) (end 149.098 80.772) (width 0.25) (layer "F.Cu") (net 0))
 (segment (start 158.242 93.218) (end 163.576 93.218) (width 0.2) (layer "F.Cu") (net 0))
 (segment (start 157.48 111.76) (end 157.48 102.108) (width 0.2) (layer "F.Cu") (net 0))
 (segment (start 128.786 66.04) (end 128.786 64.27) (width 0.25) (layer "F.Cu") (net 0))
 (segment (start 118.896 68.048) (end 144.756 68.048) (width 0.25) (layer "F.Cu") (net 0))
 (segment (start 147.32 101.6) (end 137.668 111.252) (width 0.25) (layer "F.Cu") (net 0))
 (segment (start 118.896 66.04) (end 118.896 67.842) (width 0.25) (layer "F.Cu") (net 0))
 (segment (start 146.59 64.294) (end 146.304 64.008) (width 0.25) (layer "F.Cu") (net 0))
 (segment (start 163.83 83.058) (end 157.734 83.058) (width 0.2) (layer "F.Cu") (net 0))
 (segment (start 110.03 66.04) (end 110.03 67.866) (width 0.25) (layer "F.Cu") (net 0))
 (segment (start 131.826 79.73) (end 131.09 78.994) (width 0.25) (layer "F.Cu") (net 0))
 (segment (start 129.286 70.358) (end 126.238 73.406) (width 0.25) (layer "F.Cu") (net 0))
 (segment (start 119.38 64.008) (end 119.896 64.524) (width 0.25) (layer "F.Cu") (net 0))
 (segment (start 127.786 67.842) (end 127.992 68.048) (width 0.25) (layer "F.Cu") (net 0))
 (segment (start 127.786 66.04) (end 127.786 67.842) (width 0.25) (layer "F.Cu") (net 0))
 (via (at 146.177 75.692) (size 0.8) (drill 0.4) (layers "F.Cu" "B.Cu") (free) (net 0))
 (via (at 154.94 113.919) (size 0.8) (drill 0.4) (layers "F.Cu" "B.Cu") (free) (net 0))
 (via (at 139.192 75.692) (size 0.8) (drill 0.4) (layers "F.Cu" "B.Cu") (free) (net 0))
 (via (at 148.336 108.585) (size 0.8) (drill 0.4) (layers "F.Cu" "B.Cu") (free) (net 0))
 (via (at 87.63 108.839) (size 0.8) (drill 0.4) (layers "F.Cu" "B.Cu") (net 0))
 (via (at 154.94 108.585) (size 0.8) (drill 0.4) (layers "F.Cu" "B.Cu") (free) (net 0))
 (via (at 147.574 113.919) (size 0.8) (drill 0.4) (layers "F.Cu" "B.Cu") (free) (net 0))
 (segment (start 139.7 64.643) (end 148.59 64.643) (width 0.2) (layer "B.Cu") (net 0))
 (segment (start 141.51 78.01) (end 141.51 83.09) (width 0.2) (layer "B.Cu") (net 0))
 (segment (start 149.987 92.583) (end 133.35 92.583) (width 0.2) (layer "B.Cu") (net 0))
 (segment (start 113.03 64.897) (end 113.284 64.643) (width 0.2) (layer "B.Cu") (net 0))
 (segment (start 155.575 83.566) (end 155.575 107.95) (width 0.2) (layer "B.Cu") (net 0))
 (segment (start 148.59 75.438) (end 156.464 83.312) (width 0.2) (layer "B.Cu") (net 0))
 (segment (start 137.16 86.36) (end 137.16 83.82) (width 0.2) (layer "B.Cu") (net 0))
 (segment (start 156.464 83.312) (end 156.464 112.395) (width 0.2) (layer "B.Cu") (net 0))
 (segment (start 103.251 64.262) (end 149.733 64.262) (width 0.25) (layer "B.Cu") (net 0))
 (segment (start 119.38 127) (end 167.64 127) (width 0.2) (layer "B.Cu") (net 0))
 (segment (start 139.7 64.643) (end 139.827 64.77) (width 0.2) (layer "B.Cu") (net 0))
 (segment (start 150.876 95.504) (end 149.733 94.361) (width 0.2) (layer "B.Cu") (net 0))
 (segment (start 157.978 105.908) (end 163.443 105.908) (width 0.25) (layer "B.Cu") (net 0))
 (segment (start 147.701 65.151) (end 147.59 65.262) (width 0.2) (layer "B.Cu") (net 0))
 (segment (start 104.14 111.76) (end 119.38 127) (width 0.2) (layer "B.Cu") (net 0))
 (segment (start 135.763 67.056) (end 135.89 66.929) (width 0.2) (layer "B.Cu") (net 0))
 (segment (start 140.716 71.12) (end 141.51 71.12) (width 0.25) (layer "B.Cu") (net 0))
 (segment (start 165.862 118.618) (end 167.64 116.84) (width 0.2) (layer "B.Cu") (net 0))
 (segment (start 140.716 73.279) (end 140.716 71.12) (width 0.2) (layer "B.Cu") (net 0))
 (segment (start 141.351 72.898) (end 140.843 73.406) (width 0.2) (layer "B.Cu") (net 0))
 (segment (start 146.177 106.934) (end 150.876 102.235) (width 0.2) (layer "B.Cu") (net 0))
 (segment (start 167.64 78.74) (end 166.868 77.968) (width 0.2) (layer "B.Cu") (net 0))
 (segment (start 113.03 66.04) (end 113.03 64.897) (width 0.2) (layer "B.Cu") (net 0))
 (segment (start 163.83 88.138) (end 165.862 88.138) (width 0.2) (layer "B.Cu") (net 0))
 (segment (start 121.896 64.794) (end 121.896 66.04) (width 0.2) (layer "B.Cu") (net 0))
 (segment (start 137.7 69.12) (end 137.7 66.04) (width 0.25) (layer "B.Cu") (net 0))
 (segment (start 148.336 108.585) (end 148.336 107.061) (width 0.2) (layer "B.Cu") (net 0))
 (segment (start 167.64 127) (end 167.64 78.74) (width 0.2) (layer "B.Cu") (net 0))
 (segment (start 120.896 66.921) (end 120.904 66.929) (width 0.2) (layer "B.Cu") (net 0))
 (segment (start 138.7 66.04) (end 138.7 67.04) (width 0.2) (layer "B.Cu") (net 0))
 (segment (start 157.48 86.36) (end 158.242 85.598) (width 0.25) (layer "B.Cu") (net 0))
 (segment (start 147.574 109.474) (end 146.177 108.077) (width 0.2) (layer "B.Cu") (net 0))
 (segment (start 157.988 116.078) (end 163.322 116.078) (width 0.25) (layer "B.Cu") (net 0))
 (segment (start 121.031 65.024) (end 120.896 65.159) (width 0.2) (layer "B.Cu") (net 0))
 (segment (start 157.48 96.52) (end 157.48 105.41) (width 0.25) (layer "B.Cu") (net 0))
 (segment (start 104.14 83.82) (end 104.14 111.76) (width 0.2) (layer "B.Cu") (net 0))
 (segment (start 165.862 88.138) (end 167.64 86.36) (width 0.2) (layer "B.Cu") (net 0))
 (segment (start 117.983 66.929) (end 118.11 66.802) (width 0.2) (layer "B.Cu") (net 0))
 (segment (start 154.94 91.44) (end 134.62 91.44) (width 0.2) (layer "B.Cu") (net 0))
 (segment (start 129.786 65.286) (end 129.786 66.04) (width 0.2) (layer "B.Cu") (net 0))
 (segment (start 158.242 85.598) (end 163.83 85.598) (width 0.25) (layer "B.Cu") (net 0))
 (segment (start 120.896 65.159) (end 120.896 66.04) (width 0.2) (layer "B.Cu") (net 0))
 (segment (start 156.464 112.395) (end 154.94 113.919) (width 0.2) (layer "B.Cu") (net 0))
 (segment (start 127.127 66.929) (end 127.127 65.278) (width 0.2) (layer "B.Cu") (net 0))
 (segment (start 144.399 72.898) (end 141.351 72.898) (width 0.2) (layer "B.Cu") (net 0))
 (segment (start 99.187 106.553) (end 99.187 68.326) (width 0.25) (layer "B.Cu") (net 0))
 (segment (start 129.54 71.12) (end 128.786 70.366) (width 0.25) (layer "B.Cu") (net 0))
 (segment (start 112.014 66.929) (end 117.983 66.929) (width 0.2) (layer "B.Cu") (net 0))
 (segment (start 121.92 71.12) (end 119.896 69.096) (width 0.25) (layer "B.Cu") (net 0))
 (segment (start 118.11 66.802) (end 118.11 65.151) (width 0.2) (layer "B.Cu") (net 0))
 (segment (start 138.684 65.151) (end 138.7 65.167) (width 0.2) (layer "B.Cu") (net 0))
 (segment (start 157.48 94.996) (end 157.48 86.36) (width 0.25) (layer "B.Cu") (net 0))
 (segment (start 87.63 108.839) (end 96.901 108.839) (width 0.25) (layer "B.Cu") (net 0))
 (segment (start 158.242 85.598) (end 157.48 84.836) (width 0.25) (layer "B.Cu") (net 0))
 (segment (start 148.717 64.77) (end 148.59 64.897) (width 0.2) (layer "B.Cu") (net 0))
 (segment (start 139.827 64.77) (end 139.7 64.897) (width 0.2) (layer "B.Cu") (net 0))
 (segment (start 140.843 73.406) (end 140.716 73.279) (width 0.2) (layer "B.Cu") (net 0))
 (segment (start 147.59 75.581) (end 155.575 83.566) (width 0.2) (layer "B.Cu") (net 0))
 (segment (start 149.733 94.361) (end 129.794 94.361) (width 0.2) (layer "B.Cu") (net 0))
 (segment (start 96.901 108.839) (end 99.187 106.553) (width 0.25) (layer "B.Cu") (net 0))
 (segment (start 148.336 107.061) (end 153.035 102.362) (width 0.2) (layer "B.Cu") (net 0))
 (segment (start 157.48 84.836) (end 157.48 76.2) (width 0.25) (layer "B.Cu") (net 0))
 (segment (start 153.035 102.362) (end 153.035 95.631) (width 0.2) (layer "B.Cu") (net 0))
 (segment (start 129.794 67.056) (end 135.763 67.056) (width 0.2) (layer "B.Cu") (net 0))
 (segment (start 148.59 64.897) (end 148.59 66.04) (width 0.2) (layer "B.Cu") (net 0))
 (segment (start 146.177 75.692) (end 146.177 74.676) (width 0.2) (layer "B.Cu") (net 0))
 (segment (start 137.16 83.82) (end 104.14 83.82) (width 0.2) (layer "B.Cu") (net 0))
 (segment (start 111.03 70.39) (end 111.03 66.04) (width 0.25) (layer "B.Cu") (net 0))
 (segment (start 150.876 102.235) (end 150.876 95.504) (width 0.2) (layer "B.Cu") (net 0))
 (segment (start 113.284 64.643) (end 122.047 64.643) (width 0.2) (layer "B.Cu") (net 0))
 (segment (start 127.254 65.151) (end 129.921 65.151) (width 0.2) (layer "B.Cu") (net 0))
 (segment (start 129.921 65.151) (end 129.786 65.286) (width 0.2) (layer "B.Cu") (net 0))
 (segment (start 129.786 67.048) (end 129.794 67.056) (width 0.2) (layer "B.Cu") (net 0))
 (segment (start 144.78 65.278) (end 144.907 65.151) (width 0.2) (layer "B.Cu") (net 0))
 (segment (start 163.322 118.618) (end 165.862 118.618) (width 0.2) (layer "B.Cu") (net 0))
 (segment (start 135.89 65.151) (end 138.684 65.151) (width 0.2) (layer "B.Cu") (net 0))
 (segment (start 153.035 95.631) (end 149.987 92.583) (width 0.2) (layer "B.Cu") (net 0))
 (segment (start 157.48 105.41) (end 157.48 115.57) (width 0.25) (layer "B.Cu") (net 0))
 (segment (start 148.59 64.643) (end 148.717 64.77) (width 0.2) (layer "B.Cu") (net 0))
 (segment (start 155.575 107.95) (end 154.94 108.585) (width 0.2) (layer "B.Cu") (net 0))
 (segment (start 141.51 83.09) (end 142.24 83.82) (width 0.2) (layer "B.Cu") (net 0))
 (segment (start 139.192 75.692) (end 141.51 78.01) (width 0.2) (layer "B.Cu") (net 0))
 (segment (start 112.03 66.913) (end 112.014 66.929) (width 0.2) (layer "B.Cu") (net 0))
 (segment (start 99.187 68.326) (end 103.251 64.262) (width 0.25) (layer "B.Cu") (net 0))
 (segment (start 130.81 64.643) (end 139.7 64.643) (width 0.2) (layer "B.Cu") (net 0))
 (segment (start 129.54 94.107) (end 129.54 86.36) (width 0.2) (layer "B.Cu") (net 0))
 (segment (start 157.48 115.57) (end 157.988 116.078) (width 0.25) (layer "B.Cu") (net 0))
 (segment (start 158.252 75.428) (end 163.697 75.428) (width 0.25) (layer "B.Cu") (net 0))
 (segment (start 144.907 65.151) (end 147.701 65.151) (width 0.2) (layer "B.Cu") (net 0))
 (segment (start 120.904 66.929) (end 127.127 66.929) (width 0.2) (layer "B.Cu") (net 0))
 (segment (start 158.242 95.758) (end 163.576 95.758) (width 0.25) (layer "B.Cu") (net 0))
 (segment (start 139.7 71.12) (end 137.7 69.12) (width 0.25) (layer "B.Cu") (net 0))
 (segment (start 148.59 66.04) (end 148.59 75.438) (width 0.2) (layer "B.Cu") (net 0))
 (segment (start 133.35 92.583) (end 132.08 91.313) (width 0.2) (layer "B.Cu") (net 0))
 (segment (start 157.48 72.009) (end 157.48 76.2) (width 0.25) (layer "B.Cu") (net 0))
 (segment (start 118.237 65.024) (end 121.031 65.024) (width 0.2) (layer "B.Cu") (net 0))
 (segment (start 138.7 65.167) (end 138.7 66.04) (width 0.2) (layer "B.Cu") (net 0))
 (segment (start 111.76 71.12) (end 111.03 70.39) (width 0.25) (layer "B.Cu") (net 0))
 (segment (start 147.574 113.919) (end 147.574 109.474) (width 0.2) (layer "B.Cu") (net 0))
 (segment (start 144.78 67.056) (end 144.78 65.278) (width 0.2) (layer "B.Cu") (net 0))
 (segment (start 130.81 64.643) (end 130.786 64.667) (width 0.2) (layer "B.Cu") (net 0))
 (segment (start 154.94 83.82) (end 154.94 91.44) (width 0.2) (layer "B.Cu") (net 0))
 (segment (start 165.872 108.448) (end 167.64 106.68) (width 0.2) (layer "B.Cu") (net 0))
 (segment (start 139.7 64.897) (end 139.7 66.04) (width 0.2) (layer "B.Cu") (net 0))
 (segment (start 147.59 66.04) (end 147.59 75.581) (width 0.2) (layer "B.Cu") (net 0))
 (segment (start 127.127 65.278) (end 127.254 65.151) (width 0.2) (layer "B.Cu") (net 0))
 (segment (start 111.76 71.12) (end 140.716 71.12) (width 0.25) (layer "B.Cu") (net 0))
 (segment (start 163.443 108.448) (end 165.872 108.448) (width 0.2) (layer "B.Cu") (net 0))
 (segment (start 157.48 105.41) (end 157.978 105.908) (width 0.25) (layer "B.Cu") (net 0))
 (segment (start 141.51 71.12) (end 146.59 66.04) (width 0.25) (layer "B.Cu") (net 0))
 (segment (start 129.786 66.04) (end 129.786 67.048) (width 0.2) (layer "B.Cu") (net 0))
 (segment (start 129.794 94.361) (end 129.54 94.107) (width 0.2) (layer "B.Cu") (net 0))
 (segment (start 132.08 91.313) (end 132.08 86.36) (width 0.2) (layer "B.Cu") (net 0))
 (segment (start 163.576 98.298) (end 165.862 98.298) (width 0.2) (layer "B.Cu") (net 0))
 (segment (start 112.03 66.04) (end 112.03 66.913) (width 0.2) (layer "B.Cu") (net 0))
 (segment (start 147.59 65.262) (end 147.59 66.04) (width 0.2) (layer "B.Cu") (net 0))
 (segment (start 149.733 64.262) (end 157.48 72.009) (width 0.25) (layer "B.Cu") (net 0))
 (segment (start 130.786 64.667) (end 130.786 66.04) (width 0.2) (layer "B.Cu") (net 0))
 (segment (start 135.89 66.929) (end 135.89 65.151) (width 0.2) (layer "B.Cu") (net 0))
 (segment (start 166.868 77.968) (end 163.697 77.968) (width 0.2) (layer "B.Cu") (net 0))
 (segment (start 138.7 67.04) (end 138.684 67.056) (width 0.2) (layer "B.Cu") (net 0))
 (segment (start 158.242 95.758) (end 157.48 96.52) (width 0.25) (layer "B.Cu") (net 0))
 (segment (start 120.896 66.04) (end 120.896 66.921) (width 0.2) (layer "B.Cu") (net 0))
 (segment (start 128.786 70.366) (end 128.786 66.04) (width 0.25) (layer "B.Cu") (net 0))
 (segment (start 118.11 65.151) (end 118.237 65.024) (width 0.2) (layer "B.Cu") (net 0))
 (segment (start 146.177 108.077) (end 146.177 106.934) (width 0.2) (layer "B.Cu") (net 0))
 (segment (start 165.862 98.298) (end 167.64 96.52) (width 0.2) (layer "B.Cu") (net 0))
 (segment (start 138.684 67.056) (end 144.78 67.056) (width 0.2) (layer "B.Cu") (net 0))
 (segment (start 122.047 64.643) (end 121.896 64.794) (width 0.2) (layer "B.Cu") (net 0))
 (segment (start 146.177 74.676) (end 144.399 72.898) (width 0.2) (layer "B.Cu") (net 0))
 (segment (start 122.047 64.643) (end 130.81 64.643) (width 0.2) (layer "B.Cu") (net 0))
 (segment (start 157.48 76.2) (end 158.252 75.428) (width 0.25) (layer "B.Cu") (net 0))
 (segment (start 158.242 95.758) (end 157.48 94.996) (width 0.25) (layer "B.Cu") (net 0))
 (segment (start 142.24 83.82) (end 154.94 83.82) (width 0.2) (layer "B.Cu") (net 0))
 (segment (start 134.62 91.44) (end 134.62 86.36) (width 0.2) (layer "B.Cu") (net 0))
 (segment (start 119.896 69.096) (end 119.896 66.04) (width 0.25) (layer "B.Cu") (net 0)))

